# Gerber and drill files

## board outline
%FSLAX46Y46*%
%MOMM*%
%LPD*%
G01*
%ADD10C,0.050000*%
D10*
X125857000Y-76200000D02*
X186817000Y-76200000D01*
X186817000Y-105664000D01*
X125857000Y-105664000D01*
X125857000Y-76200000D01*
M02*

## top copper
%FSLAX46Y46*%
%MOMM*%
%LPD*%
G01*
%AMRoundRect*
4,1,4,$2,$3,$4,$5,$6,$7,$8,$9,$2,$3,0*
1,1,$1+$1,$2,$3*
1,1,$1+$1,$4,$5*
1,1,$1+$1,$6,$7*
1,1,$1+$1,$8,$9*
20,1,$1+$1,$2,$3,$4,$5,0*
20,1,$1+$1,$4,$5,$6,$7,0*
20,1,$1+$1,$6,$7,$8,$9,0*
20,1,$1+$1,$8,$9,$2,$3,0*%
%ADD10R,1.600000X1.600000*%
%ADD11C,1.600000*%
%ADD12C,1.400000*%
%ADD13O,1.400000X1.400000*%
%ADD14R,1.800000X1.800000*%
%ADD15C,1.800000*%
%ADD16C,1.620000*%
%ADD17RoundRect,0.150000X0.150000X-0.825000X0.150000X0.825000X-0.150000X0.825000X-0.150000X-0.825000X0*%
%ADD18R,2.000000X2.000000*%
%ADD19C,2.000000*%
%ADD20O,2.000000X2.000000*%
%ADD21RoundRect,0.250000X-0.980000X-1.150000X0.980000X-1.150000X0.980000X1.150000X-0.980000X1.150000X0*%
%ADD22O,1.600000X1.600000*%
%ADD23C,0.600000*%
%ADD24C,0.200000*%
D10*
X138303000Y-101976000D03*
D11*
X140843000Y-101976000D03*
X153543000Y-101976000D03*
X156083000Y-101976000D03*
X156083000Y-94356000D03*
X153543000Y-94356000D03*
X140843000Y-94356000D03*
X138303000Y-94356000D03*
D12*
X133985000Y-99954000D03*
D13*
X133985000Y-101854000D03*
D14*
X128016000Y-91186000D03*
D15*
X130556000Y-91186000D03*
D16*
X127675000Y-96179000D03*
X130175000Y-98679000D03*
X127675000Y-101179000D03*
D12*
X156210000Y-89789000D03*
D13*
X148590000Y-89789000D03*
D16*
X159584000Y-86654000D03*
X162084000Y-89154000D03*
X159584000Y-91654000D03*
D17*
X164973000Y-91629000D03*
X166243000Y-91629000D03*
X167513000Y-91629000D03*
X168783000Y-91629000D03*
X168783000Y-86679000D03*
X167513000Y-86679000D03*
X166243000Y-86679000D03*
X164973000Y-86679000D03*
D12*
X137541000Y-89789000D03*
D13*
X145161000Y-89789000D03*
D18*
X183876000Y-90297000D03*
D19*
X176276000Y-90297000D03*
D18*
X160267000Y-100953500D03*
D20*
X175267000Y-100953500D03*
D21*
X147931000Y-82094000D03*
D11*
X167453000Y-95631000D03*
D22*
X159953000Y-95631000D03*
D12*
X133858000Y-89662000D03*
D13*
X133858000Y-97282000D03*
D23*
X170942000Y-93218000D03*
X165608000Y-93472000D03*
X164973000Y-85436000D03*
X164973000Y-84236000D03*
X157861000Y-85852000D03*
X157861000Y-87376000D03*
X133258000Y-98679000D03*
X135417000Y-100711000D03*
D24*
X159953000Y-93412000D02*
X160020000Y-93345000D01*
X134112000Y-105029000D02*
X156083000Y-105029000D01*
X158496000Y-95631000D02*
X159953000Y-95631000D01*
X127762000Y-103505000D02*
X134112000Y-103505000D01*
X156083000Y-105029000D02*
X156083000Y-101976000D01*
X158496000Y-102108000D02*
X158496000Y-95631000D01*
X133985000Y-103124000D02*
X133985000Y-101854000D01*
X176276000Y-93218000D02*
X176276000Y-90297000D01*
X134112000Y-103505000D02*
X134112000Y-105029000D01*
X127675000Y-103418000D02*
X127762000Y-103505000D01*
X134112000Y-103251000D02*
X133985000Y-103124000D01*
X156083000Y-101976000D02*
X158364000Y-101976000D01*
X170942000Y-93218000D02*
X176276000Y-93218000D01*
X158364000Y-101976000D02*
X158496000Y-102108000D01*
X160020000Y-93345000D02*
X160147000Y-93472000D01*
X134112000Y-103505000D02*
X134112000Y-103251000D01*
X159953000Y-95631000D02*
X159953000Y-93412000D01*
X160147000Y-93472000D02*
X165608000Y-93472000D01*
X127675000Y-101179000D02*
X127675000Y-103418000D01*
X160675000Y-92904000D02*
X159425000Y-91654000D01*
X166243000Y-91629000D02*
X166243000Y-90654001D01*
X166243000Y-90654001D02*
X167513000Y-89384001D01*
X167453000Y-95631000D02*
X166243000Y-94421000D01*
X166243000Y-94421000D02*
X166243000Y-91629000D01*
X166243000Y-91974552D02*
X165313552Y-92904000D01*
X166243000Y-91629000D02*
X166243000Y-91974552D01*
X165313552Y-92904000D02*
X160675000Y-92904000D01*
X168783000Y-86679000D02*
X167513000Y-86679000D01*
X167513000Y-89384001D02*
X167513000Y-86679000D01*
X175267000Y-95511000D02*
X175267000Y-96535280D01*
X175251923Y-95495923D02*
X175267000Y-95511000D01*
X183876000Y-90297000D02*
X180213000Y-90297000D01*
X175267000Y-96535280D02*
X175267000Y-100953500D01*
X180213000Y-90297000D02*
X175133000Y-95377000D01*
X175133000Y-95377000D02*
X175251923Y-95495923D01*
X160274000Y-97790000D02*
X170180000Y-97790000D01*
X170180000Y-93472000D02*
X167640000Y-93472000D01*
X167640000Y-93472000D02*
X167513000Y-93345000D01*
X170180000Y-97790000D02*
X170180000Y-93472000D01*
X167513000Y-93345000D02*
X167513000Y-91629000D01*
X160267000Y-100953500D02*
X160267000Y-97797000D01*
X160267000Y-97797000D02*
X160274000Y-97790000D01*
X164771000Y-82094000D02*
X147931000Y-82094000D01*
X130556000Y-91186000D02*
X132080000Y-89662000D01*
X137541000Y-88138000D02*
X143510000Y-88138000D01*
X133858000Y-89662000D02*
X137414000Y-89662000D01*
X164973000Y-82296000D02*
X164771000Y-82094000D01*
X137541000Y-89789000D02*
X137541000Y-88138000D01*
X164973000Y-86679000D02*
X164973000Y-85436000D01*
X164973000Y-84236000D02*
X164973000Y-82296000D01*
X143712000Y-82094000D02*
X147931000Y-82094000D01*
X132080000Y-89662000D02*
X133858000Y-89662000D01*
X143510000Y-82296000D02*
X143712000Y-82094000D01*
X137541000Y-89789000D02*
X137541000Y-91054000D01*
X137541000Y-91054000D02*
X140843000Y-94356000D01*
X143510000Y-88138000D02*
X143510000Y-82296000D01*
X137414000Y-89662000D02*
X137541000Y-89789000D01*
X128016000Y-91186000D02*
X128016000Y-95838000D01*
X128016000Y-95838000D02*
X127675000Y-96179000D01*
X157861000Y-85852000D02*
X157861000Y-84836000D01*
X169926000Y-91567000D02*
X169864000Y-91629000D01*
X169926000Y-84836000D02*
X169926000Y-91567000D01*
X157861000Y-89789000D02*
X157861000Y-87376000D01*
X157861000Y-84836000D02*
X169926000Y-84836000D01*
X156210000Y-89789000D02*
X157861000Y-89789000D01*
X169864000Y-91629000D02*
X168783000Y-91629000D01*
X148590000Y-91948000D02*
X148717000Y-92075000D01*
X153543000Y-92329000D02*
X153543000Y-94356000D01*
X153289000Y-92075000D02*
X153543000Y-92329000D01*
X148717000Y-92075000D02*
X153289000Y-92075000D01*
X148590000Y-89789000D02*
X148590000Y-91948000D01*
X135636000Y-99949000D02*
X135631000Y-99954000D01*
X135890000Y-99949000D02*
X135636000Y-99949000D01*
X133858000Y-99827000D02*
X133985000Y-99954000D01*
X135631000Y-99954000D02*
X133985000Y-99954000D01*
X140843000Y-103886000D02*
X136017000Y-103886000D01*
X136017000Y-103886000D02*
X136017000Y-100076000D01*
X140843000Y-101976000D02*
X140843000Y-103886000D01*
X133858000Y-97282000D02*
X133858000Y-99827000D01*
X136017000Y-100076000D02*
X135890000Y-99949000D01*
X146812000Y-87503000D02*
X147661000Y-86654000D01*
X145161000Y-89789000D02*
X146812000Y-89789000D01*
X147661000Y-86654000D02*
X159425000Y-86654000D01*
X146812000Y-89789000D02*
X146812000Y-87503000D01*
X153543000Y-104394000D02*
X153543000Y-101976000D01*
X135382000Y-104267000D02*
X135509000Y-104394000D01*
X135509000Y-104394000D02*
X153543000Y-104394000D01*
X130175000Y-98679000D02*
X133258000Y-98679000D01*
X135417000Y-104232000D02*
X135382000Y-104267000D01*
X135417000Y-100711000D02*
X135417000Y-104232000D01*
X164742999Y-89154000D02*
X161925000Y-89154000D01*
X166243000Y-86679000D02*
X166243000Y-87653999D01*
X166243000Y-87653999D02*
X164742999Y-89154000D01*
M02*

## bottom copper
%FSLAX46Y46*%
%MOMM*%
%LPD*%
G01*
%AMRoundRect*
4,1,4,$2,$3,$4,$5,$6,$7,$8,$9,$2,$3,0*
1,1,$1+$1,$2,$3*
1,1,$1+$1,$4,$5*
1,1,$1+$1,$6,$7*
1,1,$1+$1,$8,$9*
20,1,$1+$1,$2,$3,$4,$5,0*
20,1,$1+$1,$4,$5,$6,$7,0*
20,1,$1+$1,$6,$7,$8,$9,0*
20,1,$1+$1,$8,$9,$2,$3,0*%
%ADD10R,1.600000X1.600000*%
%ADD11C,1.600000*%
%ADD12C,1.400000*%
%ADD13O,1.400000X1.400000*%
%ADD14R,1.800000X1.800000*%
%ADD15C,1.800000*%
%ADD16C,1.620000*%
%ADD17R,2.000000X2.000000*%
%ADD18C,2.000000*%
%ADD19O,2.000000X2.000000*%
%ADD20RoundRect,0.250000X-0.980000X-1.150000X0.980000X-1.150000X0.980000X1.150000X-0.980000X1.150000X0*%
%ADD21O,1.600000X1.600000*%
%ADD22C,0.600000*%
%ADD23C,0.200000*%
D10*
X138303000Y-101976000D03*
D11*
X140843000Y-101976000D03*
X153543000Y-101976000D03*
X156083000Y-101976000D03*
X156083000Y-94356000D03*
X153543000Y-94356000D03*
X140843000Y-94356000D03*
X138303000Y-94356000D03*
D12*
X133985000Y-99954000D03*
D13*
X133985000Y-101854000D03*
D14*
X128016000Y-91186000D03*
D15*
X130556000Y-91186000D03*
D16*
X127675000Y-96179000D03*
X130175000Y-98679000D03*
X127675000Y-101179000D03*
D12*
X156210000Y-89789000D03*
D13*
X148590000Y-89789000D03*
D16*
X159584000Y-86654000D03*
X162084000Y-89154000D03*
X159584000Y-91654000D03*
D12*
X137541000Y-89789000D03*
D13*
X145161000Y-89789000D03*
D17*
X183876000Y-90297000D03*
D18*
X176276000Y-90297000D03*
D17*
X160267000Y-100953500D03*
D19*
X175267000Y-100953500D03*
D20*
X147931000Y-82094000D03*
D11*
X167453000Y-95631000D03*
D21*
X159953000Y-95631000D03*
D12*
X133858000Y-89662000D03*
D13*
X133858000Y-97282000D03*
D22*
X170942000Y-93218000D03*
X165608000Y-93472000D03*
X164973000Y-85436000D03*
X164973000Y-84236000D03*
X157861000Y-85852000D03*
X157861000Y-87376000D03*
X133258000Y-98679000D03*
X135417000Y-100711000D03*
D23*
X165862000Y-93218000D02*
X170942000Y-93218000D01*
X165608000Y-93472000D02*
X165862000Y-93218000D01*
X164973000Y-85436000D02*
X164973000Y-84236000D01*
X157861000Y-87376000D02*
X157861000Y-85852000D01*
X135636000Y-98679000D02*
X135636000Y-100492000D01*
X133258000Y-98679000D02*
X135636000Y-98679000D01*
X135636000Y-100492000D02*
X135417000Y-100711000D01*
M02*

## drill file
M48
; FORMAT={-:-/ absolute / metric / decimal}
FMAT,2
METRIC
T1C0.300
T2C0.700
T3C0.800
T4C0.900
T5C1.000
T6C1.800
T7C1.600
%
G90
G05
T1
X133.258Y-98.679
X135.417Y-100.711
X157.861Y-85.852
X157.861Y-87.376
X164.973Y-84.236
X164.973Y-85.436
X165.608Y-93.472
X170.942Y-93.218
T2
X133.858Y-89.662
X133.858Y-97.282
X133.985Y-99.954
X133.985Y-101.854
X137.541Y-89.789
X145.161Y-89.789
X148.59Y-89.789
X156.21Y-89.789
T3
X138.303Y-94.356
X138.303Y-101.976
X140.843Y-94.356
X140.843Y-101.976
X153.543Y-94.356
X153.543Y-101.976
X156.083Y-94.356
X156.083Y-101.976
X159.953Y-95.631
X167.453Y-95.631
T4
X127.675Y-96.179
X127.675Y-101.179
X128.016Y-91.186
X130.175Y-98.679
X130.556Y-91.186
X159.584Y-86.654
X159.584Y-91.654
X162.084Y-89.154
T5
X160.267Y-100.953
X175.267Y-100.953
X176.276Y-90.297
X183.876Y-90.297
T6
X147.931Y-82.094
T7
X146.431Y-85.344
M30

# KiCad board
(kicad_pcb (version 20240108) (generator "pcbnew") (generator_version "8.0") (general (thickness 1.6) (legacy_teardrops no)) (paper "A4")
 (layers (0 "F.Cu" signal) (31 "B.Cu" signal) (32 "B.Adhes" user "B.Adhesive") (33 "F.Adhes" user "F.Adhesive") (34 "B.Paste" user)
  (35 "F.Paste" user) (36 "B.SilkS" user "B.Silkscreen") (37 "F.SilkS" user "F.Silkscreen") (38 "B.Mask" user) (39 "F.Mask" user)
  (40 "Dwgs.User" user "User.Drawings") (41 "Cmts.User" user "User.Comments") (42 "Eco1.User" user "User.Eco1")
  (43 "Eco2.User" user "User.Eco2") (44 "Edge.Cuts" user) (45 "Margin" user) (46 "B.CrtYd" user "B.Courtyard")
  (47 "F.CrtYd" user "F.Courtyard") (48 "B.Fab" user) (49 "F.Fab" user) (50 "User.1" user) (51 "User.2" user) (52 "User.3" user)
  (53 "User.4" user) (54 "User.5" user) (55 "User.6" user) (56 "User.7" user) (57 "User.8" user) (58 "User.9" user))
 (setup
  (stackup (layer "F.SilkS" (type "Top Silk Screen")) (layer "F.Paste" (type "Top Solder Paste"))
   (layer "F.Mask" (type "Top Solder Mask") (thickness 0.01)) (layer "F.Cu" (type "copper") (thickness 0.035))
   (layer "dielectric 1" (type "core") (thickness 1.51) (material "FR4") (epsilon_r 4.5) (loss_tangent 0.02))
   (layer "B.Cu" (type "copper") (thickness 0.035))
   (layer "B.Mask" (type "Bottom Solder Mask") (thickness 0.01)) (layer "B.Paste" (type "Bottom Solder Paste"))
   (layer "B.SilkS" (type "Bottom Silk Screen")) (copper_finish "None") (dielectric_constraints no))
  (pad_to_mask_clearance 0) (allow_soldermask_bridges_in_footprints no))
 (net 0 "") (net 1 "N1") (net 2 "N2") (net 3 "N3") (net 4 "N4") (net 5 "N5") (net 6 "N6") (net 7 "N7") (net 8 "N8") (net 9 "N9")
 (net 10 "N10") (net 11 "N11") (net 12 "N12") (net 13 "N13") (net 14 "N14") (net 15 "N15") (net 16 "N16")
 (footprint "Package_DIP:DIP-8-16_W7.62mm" (layer "F.Cu") (at 138.303 101.976 90)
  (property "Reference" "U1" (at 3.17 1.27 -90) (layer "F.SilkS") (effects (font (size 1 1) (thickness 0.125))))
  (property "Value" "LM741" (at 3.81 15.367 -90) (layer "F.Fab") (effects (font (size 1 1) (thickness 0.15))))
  (pad "1" thru_hole rect (at 0 0 90) (size 1.6 1.6) (drill 0.8) (layers "*.Cu" "*.Mask") (remove_unused_layers no) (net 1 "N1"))
  (pad "2" thru_hole circle (at 0 2.54 90) (size 1.6 1.6) (drill 0.8) (layers "*.Cu" "*.Mask") (remove_unused_layers no) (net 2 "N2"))
  (pad "3" thru_hole circle (at 0 15.24 90) (size 1.6 1.6) (drill 0.8) (layers "*.Cu" "*.Mask") (remove_unused_layers no) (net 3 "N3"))
  (pad "4" thru_hole circle (at 0 17.78 90) (size 1.6 1.6) (drill 0.8) (layers "*.Cu" "*.Mask") (remove_unused_layers no) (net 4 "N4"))
  (pad "5" thru_hole circle (at 7.62 17.78 90) (size 1.6 1.6) (drill 0.8) (layers "*.Cu" "*.Mask") (remove_unused_layers no) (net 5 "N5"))
  (pad "6" thru_hole circle (at 7.62 15.24 90) (size 1.6 1.6) (drill 0.8) (layers "*.Cu" "*.Mask") (remove_unused_layers no) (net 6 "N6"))
  (pad "7" thru_hole circle (at 7.62 2.54 90) (size 1.6 1.6) (drill 0.8) (layers "*.Cu" "*.Mask") (remove_unused_layers no) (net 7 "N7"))
  (pad "8" thru_hole circle (at 7.62 0 90) (size 1.6 1.6) (drill 0.8) (layers "*.Cu" "*.Mask") (remove_unused_layers no) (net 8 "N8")))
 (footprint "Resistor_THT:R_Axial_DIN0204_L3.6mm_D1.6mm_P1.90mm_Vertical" (layer "F.Cu") (at 133.985 99.954 -90)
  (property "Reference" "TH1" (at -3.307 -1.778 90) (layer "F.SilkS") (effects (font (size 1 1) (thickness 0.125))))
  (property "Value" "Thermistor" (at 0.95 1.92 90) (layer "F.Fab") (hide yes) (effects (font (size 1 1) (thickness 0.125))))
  (pad "1" thru_hole circle (at 0 0 270) (size 1.4 1.4) (drill 0.7) (layers "*.Cu" "*.Mask") (remove_unused_layers no) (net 2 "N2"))
  (pad "2" thru_hole oval (at 1.9 0 270) (size 1.4 1.4) (drill 0.7) (layers "*.Cu" "*.Mask") (remove_unused_layers no) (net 4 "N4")))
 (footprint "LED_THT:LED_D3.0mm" (layer "F.Cu") (at 128.016 91.186)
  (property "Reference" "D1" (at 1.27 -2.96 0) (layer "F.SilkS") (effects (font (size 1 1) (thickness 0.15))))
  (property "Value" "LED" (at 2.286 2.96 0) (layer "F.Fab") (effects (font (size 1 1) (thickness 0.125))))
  (pad "1" thru_hole rect (at 0 0) (size 1.8 1.8) (drill 0.9) (layers "*.Cu" "*.Mask") (remove_unused_layers no) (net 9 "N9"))
  (pad "2" thru_hole circle (at 2.54 0) (size 1.8 1.8) (drill 0.9) (layers "*.Cu" "*.Mask") (remove_unused_layers no) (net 7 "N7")))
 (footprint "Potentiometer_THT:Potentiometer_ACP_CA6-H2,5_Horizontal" (layer "F.Cu") (at 127.675 96.179)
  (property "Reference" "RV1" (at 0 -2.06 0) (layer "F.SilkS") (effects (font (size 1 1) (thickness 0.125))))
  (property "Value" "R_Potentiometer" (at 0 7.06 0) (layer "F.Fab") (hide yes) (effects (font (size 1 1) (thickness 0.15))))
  (pad "1" thru_hole circle (at 0 0) (size 1.62 1.62) (drill 0.9) (layers "*.Cu" "*.Mask") (remove_unused_layers no) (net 9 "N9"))
  (pad "2" thru_hole circle (at 2.5 2.5) (size 1.62 1.62) (drill 0.9) (layers "*.Cu" "*.Mask") (remove_unused_layers no) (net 3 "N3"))
  (pad "3" thru_hole circle (at 0 5) (size 1.62 1.62) (drill 0.9) (layers "*.Cu" "*.Mask") (remove_unused_layers no) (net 4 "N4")))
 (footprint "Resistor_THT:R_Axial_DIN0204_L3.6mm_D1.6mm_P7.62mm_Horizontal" (layer "F.Cu") (at 156.21 89.789 180)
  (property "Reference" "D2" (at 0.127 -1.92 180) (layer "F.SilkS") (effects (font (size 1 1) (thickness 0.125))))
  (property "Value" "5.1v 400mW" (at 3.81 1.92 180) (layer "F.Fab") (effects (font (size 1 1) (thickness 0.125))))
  (pad "1" thru_hole circle (at 0 0 180) (size 1.4 1.4) (drill 0.7) (layers "*.Cu" "*.Mask") (remove_unused_layers no) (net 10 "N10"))
  (pad "2" thru_hole oval (at 7.62 0 180) (size 1.4 1.4) (drill 0.7) (layers "*.Cu" "*.Mask") (remove_unused_layers no) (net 6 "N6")))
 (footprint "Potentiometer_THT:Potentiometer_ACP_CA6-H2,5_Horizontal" (layer "F.Cu") (at 159.584 86.654)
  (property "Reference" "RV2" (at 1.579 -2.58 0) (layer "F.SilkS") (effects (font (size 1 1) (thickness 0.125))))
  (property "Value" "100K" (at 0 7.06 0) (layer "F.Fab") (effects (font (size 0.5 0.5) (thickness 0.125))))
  (pad "1" thru_hole circle (at 0 0) (size 1.62 1.62) (drill 0.9) (layers "*.Cu" "*.Mask") (remove_unused_layers no) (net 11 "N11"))
  (pad "2" thru_hole circle (at 2.5 2.5) (size 1.62 1.62) (drill 0.9) (layers "*.Cu" "*.Mask") (remove_unused_layers no) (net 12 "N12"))
  (pad "3" thru_hole circle (at 0 5) (size 1.62 1.62) (drill 0.9) (layers "*.Cu" "*.Mask") (remove_unused_layers no) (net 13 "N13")))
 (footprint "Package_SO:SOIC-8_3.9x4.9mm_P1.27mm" (layer "F.Cu") (at 166.878 89.154 90)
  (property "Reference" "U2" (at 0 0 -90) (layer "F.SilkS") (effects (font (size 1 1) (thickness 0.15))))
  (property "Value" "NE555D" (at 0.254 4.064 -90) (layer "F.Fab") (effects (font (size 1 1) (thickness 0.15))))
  (pad "1" smd roundrect (at -2.475 -1.905 90) (size 1.95 0.6) (layers "F.Cu" "F.Paste" "F.Mask") (roundrect_rratio 0.25) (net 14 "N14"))
  (pad "2" smd roundrect (at -2.475 -0.635 90) (size 1.95 0.6) (layers "F.Cu" "F.Paste" "F.Mask") (roundrect_rratio 0.25) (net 13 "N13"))
  (pad "3" smd roundrect (at -2.475 0.635 90) (size 1.95 0.6) (layers "F.Cu" "F.Paste" "F.Mask") (roundrect_rratio 0.25) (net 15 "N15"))
  (pad "4" smd roundrect (at -2.475 1.905 90) (size 1.95 0.6) (layers "F.Cu" "F.Paste" "F.Mask") (roundrect_rratio 0.25) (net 10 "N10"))
  (pad "5" smd roundrect (at 2.475 1.905 90) (size 1.95 0.6) (layers "F.Cu" "F.Paste" "F.Mask") (roundrect_rratio 0.25) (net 13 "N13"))
  (pad "6" smd roundrect (at 2.475 0.635 90) (size 1.95 0.6) (layers "F.Cu" "F.Paste" "F.Mask") (roundrect_rratio 0.25) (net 13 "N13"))
  (pad "7" smd roundrect (at 2.475 -0.635 90) (size 1.95 0.6) (layers "F.Cu" "F.Paste" "F.Mask") (roundrect_rratio 0.25) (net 12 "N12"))
  (pad "8" smd roundrect (at 2.475 -1.905 90) (size 1.95 0.6) (layers "F.Cu" "F.Paste" "F.Mask") (roundrect_rratio 0.25) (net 7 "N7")))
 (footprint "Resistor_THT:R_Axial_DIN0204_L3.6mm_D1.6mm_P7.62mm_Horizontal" (layer "F.Cu") (at 137.541 89.789)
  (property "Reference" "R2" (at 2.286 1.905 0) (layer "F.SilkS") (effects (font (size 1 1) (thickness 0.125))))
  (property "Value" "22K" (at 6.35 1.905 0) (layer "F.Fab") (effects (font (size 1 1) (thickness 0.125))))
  (pad "1" thru_hole circle (at 0 0) (size 1.4 1.4) (drill 0.7) (layers "*.Cu" "*.Mask") (remove_unused_layers no) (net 7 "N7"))
  (pad "2" thru_hole oval (at 7.62 0) (size 1.4 1.4) (drill 0.7) (layers "*.Cu" "*.Mask") (remove_unused_layers no) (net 11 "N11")))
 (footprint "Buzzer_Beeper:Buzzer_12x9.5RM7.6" (layer "F.Cu") (at 183.876 90.297 180)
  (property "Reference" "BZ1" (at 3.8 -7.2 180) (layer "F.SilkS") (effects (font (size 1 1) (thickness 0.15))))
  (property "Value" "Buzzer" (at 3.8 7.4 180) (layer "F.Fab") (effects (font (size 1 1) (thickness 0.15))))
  (pad "1" thru_hole rect (at 0 0 180) (size 2 2) (drill 1) (layers "*.Cu" "*.Mask") (remove_unused_layers no) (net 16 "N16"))
  (pad "2" thru_hole circle (at 7.6 0 180) (size 2 2) (drill 1) (layers "*.Cu" "*.Mask") (remove_unused_layers no) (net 4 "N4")))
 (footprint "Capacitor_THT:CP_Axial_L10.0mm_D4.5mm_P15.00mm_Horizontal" (layer "F.Cu") (at 160.267 100.9535)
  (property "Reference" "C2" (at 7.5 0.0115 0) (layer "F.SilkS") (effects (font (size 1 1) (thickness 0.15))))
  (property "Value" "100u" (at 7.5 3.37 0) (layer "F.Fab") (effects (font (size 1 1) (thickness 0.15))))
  (pad "1" thru_hole rect (at 0 0) (size 2 2) (drill 1) (layers "*.Cu" "*.Mask") (remove_unused_layers no) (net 15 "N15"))
  (pad "2" thru_hole oval (at 15 0) (size 2 2) (drill 1) (layers "*.Cu" "*.Mask") (remove_unused_layers no) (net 16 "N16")))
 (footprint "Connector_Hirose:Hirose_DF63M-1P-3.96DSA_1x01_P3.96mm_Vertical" (layer "F.Cu") (at 147.931 82.094)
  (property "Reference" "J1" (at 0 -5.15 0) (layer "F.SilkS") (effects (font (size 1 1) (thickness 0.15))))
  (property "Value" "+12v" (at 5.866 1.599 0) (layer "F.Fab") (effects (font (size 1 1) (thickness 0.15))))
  (pad "" np_thru_hole circle (at -1.5 3.25) (size 1.6 1.6) (drill 1.6) (layers "*.Cu" "*.Mask"))
  (pad "1" thru_hole roundrect (at 0 0) (size 2.46 2.8) (drill 1.8) (layers "*.Cu" "*.Mask") (remove_unused_layers no)
   (roundrect_rratio 0.101626) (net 7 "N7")))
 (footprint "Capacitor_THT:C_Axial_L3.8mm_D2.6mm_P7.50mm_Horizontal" (layer "F.Cu") (at 167.453 95.631 180)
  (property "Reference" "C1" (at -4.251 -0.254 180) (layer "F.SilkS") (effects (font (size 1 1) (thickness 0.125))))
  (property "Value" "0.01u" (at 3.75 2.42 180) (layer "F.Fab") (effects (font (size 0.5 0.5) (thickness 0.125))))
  (pad "1" thru_hole circle (at 0 0 180) (size 1.6 1.6) (drill 0.8) (layers "*.Cu" "*.Mask") (remove_unused_layers no) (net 13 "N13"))
  (pad "2" thru_hole oval (at 7.5 0 180) (size 1.6 1.6) (drill 0.8) (layers "*.Cu" "*.Mask") (remove_unused_layers no) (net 4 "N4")))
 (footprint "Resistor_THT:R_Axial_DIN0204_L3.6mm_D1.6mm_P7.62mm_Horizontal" (layer "F.Cu") (at 133.858 89.662 -90)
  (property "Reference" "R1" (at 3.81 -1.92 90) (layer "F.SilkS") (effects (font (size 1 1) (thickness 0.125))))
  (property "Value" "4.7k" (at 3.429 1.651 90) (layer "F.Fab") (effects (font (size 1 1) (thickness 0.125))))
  (pad "1" thru_hole circle (at 0 0 270) (size 1.4 1.4) (drill 0.7) (layers "*.Cu" "*.Mask") (remove_unused_layers no) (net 7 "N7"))
  (pad "2" thru_hole oval (at 7.62 0 270) (size 1.4 1.4) (drill 0.7) (layers "*.Cu" "*.Mask") (remove_unused_layers no) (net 2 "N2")))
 (gr_rect (start 125.857 76.2) (end 186.817 105.664) (stroke (width 0.05) (type default)) (fill none) (layer "Edge.Cuts"))
 (segment (start 159.953 93.412) (end 160.02 93.345) (width 0.2) (layer "F.Cu") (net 4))
 (segment (start 134.112 105.029) (end 156.083 105.029) (width 0.2) (layer "F.Cu") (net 4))
 (segment (start 158.496 95.631) (end 159.953 95.631) (width 0.2) (layer "F.Cu") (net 4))
 (segment (start 127.762 103.505) (end 134.112 103.505) (width 0.2) (layer "F.Cu") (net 4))
 (segment (start 156.083 105.029) (end 156.083 101.976) (width 0.2) (layer "F.Cu") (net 4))
 (segment (start 158.496 102.108) (end 158.496 95.631) (width 0.2) (layer "F.Cu") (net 4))
 (segment (start 133.985 103.124) (end 133.985 101.854) (width 0.2) (layer "F.Cu") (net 4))
 (segment (start 176.276 93.218) (end 176.276 90.297) (width 0.2) (layer "F.Cu") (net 4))
 (segment (start 134.112 103.505) (end 134.112 105.029) (width 0.2) (layer "F.Cu") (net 4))
 (segment (start 127.675 103.418) (end 127.762 103.505) (width 0.2) (layer "F.Cu") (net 4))
 (segment (start 134.112 103.251) (end 133.985 103.124) (width 0.2) (layer "F.Cu") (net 4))
 (segment (start 156.083 101.976) (end 158.364 101.976) (width 0.2) (layer "F.Cu") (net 4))
 (segment (start 170.942 93.218) (end 176.276 93.218) (width 0.2) (layer "F.Cu") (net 4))
 (segment (start 158.364 101.976) (end 158.496 102.108) (width 0.2) (layer "F.Cu") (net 4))
 (segment (start 160.02 93.345) (end 160.147 93.472) (width 0.2) (layer "F.Cu") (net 4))
 (segment (start 134.112 103.505) (end 134.112 103.251) (width 0.2) (layer "F.Cu") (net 4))
 (segment (start 159.953 95.631) (end 159.953 93.412) (width 0.2) (layer "F.Cu") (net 4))
 (segment (start 160.147 93.472) (end 165.608 93.472) (width 0.2) (layer "F.Cu") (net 4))
 (segment (start 127.675 101.179) (end 127.675 103.418) (width 0.2) (layer "F.Cu") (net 4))
 (via (at 170.942 93.218) (size 0.6) (drill 0.3) (layers "F.Cu" "B.Cu") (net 4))
 (via (at 165.608 93.472) (size 0.6) (drill 0.3) (layers "F.Cu" "B.Cu") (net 4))
 (segment (start 165.862 93.218) (end 170.942 93.218) (width 0.2) (layer "B.Cu") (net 4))
 (segment (start 165.608 93.472) (end 165.862 93.218) (width 0.2) (layer "B.Cu") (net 4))
 (segment (start 160.675 92.904) (end 159.425 91.654) (width 0.2) (layer "F.Cu") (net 13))
 (segment (start 166.243 91.629) (end 166.243 90.654001) (width 0.2) (layer "F.Cu") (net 13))
 (segment (start 166.243 90.654001) (end 167.513 89.384001) (width 0.2) (layer "F.Cu") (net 13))
 (segment (start 167.453 95.631) (end 166.243 94.421) (width 0.2) (layer "F.Cu") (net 13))
 (segment (start 166.243 94.421) (end 166.243 91.629) (width 0.2) (layer "F.Cu") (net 13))
 (segment (start 166.243 91.974552) (end 165.313552 92.904) (width 0.2) (layer "F.Cu") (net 13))
 (segment (start 166.243 91.629) (end 166.243 91.974552) (width 0.2) (layer "F.Cu") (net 13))
 (segment (start 165.313552 92.904) (end 160.675 92.904) (width 0.2) (layer "F.Cu") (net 13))
 (segment (start 168.783 86.679) (end 167.513 86.679) (width 0.2) (layer "F.Cu") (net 13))
 (segment (start 167.513 89.384001) (end 167.513 86.679) (width 0.2) (layer "F.Cu") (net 13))
 (segment (start 175.267 95.511) (end 175.267 96.53528) (width 0.2) (layer "F.Cu") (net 16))
 (segment (start 175.251923 95.495923) (end 175.267 95.511) (width 0.2) (layer "F.Cu") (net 16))
 (segment (start 183.876 90.297) (end 180.213 90.297) (width 0.2) (layer "F.Cu") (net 16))
 (segment (start 175.267 96.53528) (end 175.267 100.9535) (width 0.2) (layer "F.Cu") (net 16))
 (segment (start 180.213 90.297) (end 175.133 95.377) (width 0.2) (layer "F.Cu") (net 16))
 (segment (start 175.133 95.377) (end 175.251923 95.495923) (width 0.2) (layer "F.Cu") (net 16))
 (segment (start 160.274 97.79) (end 170.18 97.79) (width 0.2) (layer "F.Cu") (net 15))
 (segment (start 170.18 93.472) (end 167.64 93.472) (width 0.2) (layer "F.Cu") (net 15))
 (segment (start 167.64 93.472) (end 167.513 93.345) (width 0.2) (layer "F.Cu") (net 15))
 (segment (start 170.18 97.79) (end 170.18 93.472) (width 0.2) (layer "F.Cu") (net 15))
 (segment (start 167.513 93.345) (end 167.513 91.629) (width 0.2) (layer "F.Cu") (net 15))
 (segment (start 160.267 100.9535) (end 160.267 97.797) (width 0.2) (layer "F.Cu") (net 15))
 (segment (start 160.267 97.797) (end 160.274 97.79) (width 0.2) (layer "F.Cu") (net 15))
 (segment (start 164.771 82.094) (end 147.931 82.094) (width 0.2) (layer "F.Cu") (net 7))
 (segment (start 130.556 91.186) (end 132.08 89.662) (width 0.2) (layer "F.Cu") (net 7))
 (segment (start 137.541 88.138) (end 143.51 88.138) (width 0.2) (layer "F.Cu") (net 7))
 (segment (start 133.858 89.662) (end 137.414 89.662) (width 0.2) (layer "F.Cu") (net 7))
 (segment (start 164.973 82.296) (end 164.771 82.094) (width 0.2) (layer "F.Cu") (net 7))
 (segment (start 137.541 89.789) (end 137.541 88.138) (width 0.2) (layer "F.Cu") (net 7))
 (segment (start 164.973 86.679) (end 164.973 85.436) (width 0.2) (layer "F.Cu") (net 7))
 (segment (start 164.973 84.236) (end 164.973 82.296) (width 0.2) (layer "F.Cu") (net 7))
 (segment (start 143.712 82.094) (end 147.931 82.094) (width 0.2) (layer "F.Cu") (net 7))
 (segment (start 132.08 89.662) (end 133.858 89.662) (width 0.2) (layer "F.Cu") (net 7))
 (segment (start 143.51 82.296) (end 143.712 82.094) (width 0.2) (layer "F.Cu") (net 7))
 (segment (start 137.541 89.789) (end 137.541 91.054) (width 0.2) (layer "F.Cu") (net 7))
 (segment (start 137.541 91.054) (end 140.843 94.356) (width 0.2) (layer "F.Cu") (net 7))
 (segment (start 143.51 88.138) (end 143.51 82.296) (width 0.2) (layer "F.Cu") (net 7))
 (segment (start 137.414 89.662) (end 137.541 89.789) (width 0.2) (layer "F.Cu") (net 7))
 (via (at 164.973 85.436) (size 0.6) (drill 0.3) (layers "F.Cu" "B.Cu") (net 7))
 (via (at 164.973 84.236) (size 0.6) (drill 0.3) (layers "F.Cu" "B.Cu") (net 7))
 (segment (start 164.973 85.436) (end 164.973 84.236) (width 0.2) (layer "B.Cu") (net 7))
 (segment (start 128.016 91.186) (end 128.016 95.838) (width 0.2) (layer "F.Cu") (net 9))
 (segment (start 128.016 95.838) (end 127.675 96.179) (width 0.2) (layer "F.Cu") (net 9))
 (segment (start 157.861 85.852) (end 157.861 84.836) (width 0.2) (layer "F.Cu") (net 10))
 (segment (start 169.926 91.567) (end 169.864 91.629) (width 0.2) (layer "F.Cu") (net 10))
 (segment (start 169.926 84.836) (end 169.926 91.567) (width 0.2) (layer "F.Cu") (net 10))
 (segment (start 157.861 89.789) (end 157.861 87.376) (width 0.2) (layer "F.Cu") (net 10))
 (segment (start 157.861 84.836) (end 169.926 84.836) (width 0.2) (layer "F.Cu") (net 10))
 (segment (start 156.21 89.789) (end 157.861 89.789) (width 0.2) (layer "F.Cu") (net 10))
 (segment (start 169.864 91.629) (end 168.783 91.629) (width 0.2) (layer "F.Cu") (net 10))
 (via (at 157.861 85.852) (size 0.6) (drill 0.3) (layers "F.Cu" "B.Cu") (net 10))
 (via (at 157.861 87.376) (size 0.6) (drill 0.3) (layers "F.Cu" "B.Cu") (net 10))
 (segment (start 157.861 87.376) (end 157.861 85.852) (width 0.2) (layer "B.Cu") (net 10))
 (segment (start 148.59 91.948) (end 148.717 92.075) (width 0.2) (layer "F.Cu") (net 6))
 (segment (start 153.543 92.329) (end 153.543 94.356) (width 0.2) (layer "F.Cu") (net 6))
 (segment (start 153.289 92.075) (end 153.543 92.329) (width 0.2) (layer "F.Cu") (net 6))
 (segment (start 148.717 92.075) (end 153.289 92.075) (width 0.2) (layer "F.Cu") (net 6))
 (segment (start 148.59 89.789) (end 148.59 91.948) (width 0.2) (layer "F.Cu") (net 6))
 (segment (start 135.636 99.949) (end 135.631 99.954) (width 0.2) (layer "F.Cu") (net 2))
 (segment (start 135.89 99.949) (end 135.636 99.949) (width 0.2) (layer "F.Cu") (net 2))
 (segment (start 133.858 99.827) (end 133.985 99.954) (width 0.2) (layer "F.Cu") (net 2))
 (segment (start 135.631 99.954) (end 133.985 99.954) (width 0.2) (layer "F.Cu") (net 2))
 (segment (start 140.843 103.886) (end 136.017 103.886) (width 0.2) (layer "F.Cu") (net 2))
 (segment (start 136.017 103.886) (end 136.017 100.076) (width 0.2) (layer "F.Cu") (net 2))
 (segment (start 140.843 101.976) (end 140.843 103.886) (width 0.2) (layer "F.Cu") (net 2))
 (segment (start 133.858 97.282) (end 133.858 99.827) (width 0.2) (layer "F.Cu") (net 2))
 (segment (start 136.017 100.076) (end 135.89 99.949) (width 0.2) (layer "F.Cu") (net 2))
 (segment (start 146.812 87.503) (end 147.661 86.654) (width 0.2) (layer "F.Cu") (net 11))
 (segment (start 145.161 89.789) (end 146.812 89.789) (width 0.2) (layer "F.Cu") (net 11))
 (segment (start 147.661 86.654) (end 159.425 86.654) (width 0.2) (layer "F.Cu") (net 11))
 (segment (start 146.812 89.789) (end 146.812 87.503) (width 0.2) (layer "F.Cu") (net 11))
 (segment (start 153.543 104.394) (end 153.543 101.976) (width 0.2) (layer "F.Cu") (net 3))
 (segment (start 135.382 104.267) (end 135.509 104.394) (width 0.2) (layer "F.Cu") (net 3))
 (segment (start 135.509 104.394) (end 153.543 104.394) (width 0.2) (layer "F.Cu") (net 3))
 (segment (start 130.175 98.679) (end 133.258 98.679) (width 0.2) (layer "F.Cu") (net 3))
 (segment (start 135.417 104.232) (end 135.382 104.267) (width 0.2) (layer "F.Cu") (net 3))
 (segment (start 135.417 100.711) (end 135.417 104.232) (width 0.2) (layer "F.Cu") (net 3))
 (via (at 133.258 98.679) (size 0.6) (drill 0.3) (layers "F.Cu" "B.Cu") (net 3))
 (via (at 135.417 100.711) (size 0.6) (drill 0.3) (layers "F.Cu" "B.Cu") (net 3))
 (segment (start 135.636 98.679) (end 135.636 100.492) (width 0.2) (layer "B.Cu") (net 3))
 (segment (start 133.258 98.679) (end 135.636 98.679) (width 0.2) (layer "B.Cu") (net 3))
 (segment (start 135.636 100.492) (end 135.417 100.711) (width 0.2) (layer "B.Cu") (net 3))
 (segment (start 164.742999 89.154) (end 161.925 89.154) (width 0.2) (layer "F.Cu") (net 12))
 (segment (start 166.243 86.679) (end 166.243 87.653999) (width 0.2) (layer "F.Cu") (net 12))
 (segment (start 166.243 87.653999) (end 164.742999 89.154) (width 0.2) (layer "F.Cu") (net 12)))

